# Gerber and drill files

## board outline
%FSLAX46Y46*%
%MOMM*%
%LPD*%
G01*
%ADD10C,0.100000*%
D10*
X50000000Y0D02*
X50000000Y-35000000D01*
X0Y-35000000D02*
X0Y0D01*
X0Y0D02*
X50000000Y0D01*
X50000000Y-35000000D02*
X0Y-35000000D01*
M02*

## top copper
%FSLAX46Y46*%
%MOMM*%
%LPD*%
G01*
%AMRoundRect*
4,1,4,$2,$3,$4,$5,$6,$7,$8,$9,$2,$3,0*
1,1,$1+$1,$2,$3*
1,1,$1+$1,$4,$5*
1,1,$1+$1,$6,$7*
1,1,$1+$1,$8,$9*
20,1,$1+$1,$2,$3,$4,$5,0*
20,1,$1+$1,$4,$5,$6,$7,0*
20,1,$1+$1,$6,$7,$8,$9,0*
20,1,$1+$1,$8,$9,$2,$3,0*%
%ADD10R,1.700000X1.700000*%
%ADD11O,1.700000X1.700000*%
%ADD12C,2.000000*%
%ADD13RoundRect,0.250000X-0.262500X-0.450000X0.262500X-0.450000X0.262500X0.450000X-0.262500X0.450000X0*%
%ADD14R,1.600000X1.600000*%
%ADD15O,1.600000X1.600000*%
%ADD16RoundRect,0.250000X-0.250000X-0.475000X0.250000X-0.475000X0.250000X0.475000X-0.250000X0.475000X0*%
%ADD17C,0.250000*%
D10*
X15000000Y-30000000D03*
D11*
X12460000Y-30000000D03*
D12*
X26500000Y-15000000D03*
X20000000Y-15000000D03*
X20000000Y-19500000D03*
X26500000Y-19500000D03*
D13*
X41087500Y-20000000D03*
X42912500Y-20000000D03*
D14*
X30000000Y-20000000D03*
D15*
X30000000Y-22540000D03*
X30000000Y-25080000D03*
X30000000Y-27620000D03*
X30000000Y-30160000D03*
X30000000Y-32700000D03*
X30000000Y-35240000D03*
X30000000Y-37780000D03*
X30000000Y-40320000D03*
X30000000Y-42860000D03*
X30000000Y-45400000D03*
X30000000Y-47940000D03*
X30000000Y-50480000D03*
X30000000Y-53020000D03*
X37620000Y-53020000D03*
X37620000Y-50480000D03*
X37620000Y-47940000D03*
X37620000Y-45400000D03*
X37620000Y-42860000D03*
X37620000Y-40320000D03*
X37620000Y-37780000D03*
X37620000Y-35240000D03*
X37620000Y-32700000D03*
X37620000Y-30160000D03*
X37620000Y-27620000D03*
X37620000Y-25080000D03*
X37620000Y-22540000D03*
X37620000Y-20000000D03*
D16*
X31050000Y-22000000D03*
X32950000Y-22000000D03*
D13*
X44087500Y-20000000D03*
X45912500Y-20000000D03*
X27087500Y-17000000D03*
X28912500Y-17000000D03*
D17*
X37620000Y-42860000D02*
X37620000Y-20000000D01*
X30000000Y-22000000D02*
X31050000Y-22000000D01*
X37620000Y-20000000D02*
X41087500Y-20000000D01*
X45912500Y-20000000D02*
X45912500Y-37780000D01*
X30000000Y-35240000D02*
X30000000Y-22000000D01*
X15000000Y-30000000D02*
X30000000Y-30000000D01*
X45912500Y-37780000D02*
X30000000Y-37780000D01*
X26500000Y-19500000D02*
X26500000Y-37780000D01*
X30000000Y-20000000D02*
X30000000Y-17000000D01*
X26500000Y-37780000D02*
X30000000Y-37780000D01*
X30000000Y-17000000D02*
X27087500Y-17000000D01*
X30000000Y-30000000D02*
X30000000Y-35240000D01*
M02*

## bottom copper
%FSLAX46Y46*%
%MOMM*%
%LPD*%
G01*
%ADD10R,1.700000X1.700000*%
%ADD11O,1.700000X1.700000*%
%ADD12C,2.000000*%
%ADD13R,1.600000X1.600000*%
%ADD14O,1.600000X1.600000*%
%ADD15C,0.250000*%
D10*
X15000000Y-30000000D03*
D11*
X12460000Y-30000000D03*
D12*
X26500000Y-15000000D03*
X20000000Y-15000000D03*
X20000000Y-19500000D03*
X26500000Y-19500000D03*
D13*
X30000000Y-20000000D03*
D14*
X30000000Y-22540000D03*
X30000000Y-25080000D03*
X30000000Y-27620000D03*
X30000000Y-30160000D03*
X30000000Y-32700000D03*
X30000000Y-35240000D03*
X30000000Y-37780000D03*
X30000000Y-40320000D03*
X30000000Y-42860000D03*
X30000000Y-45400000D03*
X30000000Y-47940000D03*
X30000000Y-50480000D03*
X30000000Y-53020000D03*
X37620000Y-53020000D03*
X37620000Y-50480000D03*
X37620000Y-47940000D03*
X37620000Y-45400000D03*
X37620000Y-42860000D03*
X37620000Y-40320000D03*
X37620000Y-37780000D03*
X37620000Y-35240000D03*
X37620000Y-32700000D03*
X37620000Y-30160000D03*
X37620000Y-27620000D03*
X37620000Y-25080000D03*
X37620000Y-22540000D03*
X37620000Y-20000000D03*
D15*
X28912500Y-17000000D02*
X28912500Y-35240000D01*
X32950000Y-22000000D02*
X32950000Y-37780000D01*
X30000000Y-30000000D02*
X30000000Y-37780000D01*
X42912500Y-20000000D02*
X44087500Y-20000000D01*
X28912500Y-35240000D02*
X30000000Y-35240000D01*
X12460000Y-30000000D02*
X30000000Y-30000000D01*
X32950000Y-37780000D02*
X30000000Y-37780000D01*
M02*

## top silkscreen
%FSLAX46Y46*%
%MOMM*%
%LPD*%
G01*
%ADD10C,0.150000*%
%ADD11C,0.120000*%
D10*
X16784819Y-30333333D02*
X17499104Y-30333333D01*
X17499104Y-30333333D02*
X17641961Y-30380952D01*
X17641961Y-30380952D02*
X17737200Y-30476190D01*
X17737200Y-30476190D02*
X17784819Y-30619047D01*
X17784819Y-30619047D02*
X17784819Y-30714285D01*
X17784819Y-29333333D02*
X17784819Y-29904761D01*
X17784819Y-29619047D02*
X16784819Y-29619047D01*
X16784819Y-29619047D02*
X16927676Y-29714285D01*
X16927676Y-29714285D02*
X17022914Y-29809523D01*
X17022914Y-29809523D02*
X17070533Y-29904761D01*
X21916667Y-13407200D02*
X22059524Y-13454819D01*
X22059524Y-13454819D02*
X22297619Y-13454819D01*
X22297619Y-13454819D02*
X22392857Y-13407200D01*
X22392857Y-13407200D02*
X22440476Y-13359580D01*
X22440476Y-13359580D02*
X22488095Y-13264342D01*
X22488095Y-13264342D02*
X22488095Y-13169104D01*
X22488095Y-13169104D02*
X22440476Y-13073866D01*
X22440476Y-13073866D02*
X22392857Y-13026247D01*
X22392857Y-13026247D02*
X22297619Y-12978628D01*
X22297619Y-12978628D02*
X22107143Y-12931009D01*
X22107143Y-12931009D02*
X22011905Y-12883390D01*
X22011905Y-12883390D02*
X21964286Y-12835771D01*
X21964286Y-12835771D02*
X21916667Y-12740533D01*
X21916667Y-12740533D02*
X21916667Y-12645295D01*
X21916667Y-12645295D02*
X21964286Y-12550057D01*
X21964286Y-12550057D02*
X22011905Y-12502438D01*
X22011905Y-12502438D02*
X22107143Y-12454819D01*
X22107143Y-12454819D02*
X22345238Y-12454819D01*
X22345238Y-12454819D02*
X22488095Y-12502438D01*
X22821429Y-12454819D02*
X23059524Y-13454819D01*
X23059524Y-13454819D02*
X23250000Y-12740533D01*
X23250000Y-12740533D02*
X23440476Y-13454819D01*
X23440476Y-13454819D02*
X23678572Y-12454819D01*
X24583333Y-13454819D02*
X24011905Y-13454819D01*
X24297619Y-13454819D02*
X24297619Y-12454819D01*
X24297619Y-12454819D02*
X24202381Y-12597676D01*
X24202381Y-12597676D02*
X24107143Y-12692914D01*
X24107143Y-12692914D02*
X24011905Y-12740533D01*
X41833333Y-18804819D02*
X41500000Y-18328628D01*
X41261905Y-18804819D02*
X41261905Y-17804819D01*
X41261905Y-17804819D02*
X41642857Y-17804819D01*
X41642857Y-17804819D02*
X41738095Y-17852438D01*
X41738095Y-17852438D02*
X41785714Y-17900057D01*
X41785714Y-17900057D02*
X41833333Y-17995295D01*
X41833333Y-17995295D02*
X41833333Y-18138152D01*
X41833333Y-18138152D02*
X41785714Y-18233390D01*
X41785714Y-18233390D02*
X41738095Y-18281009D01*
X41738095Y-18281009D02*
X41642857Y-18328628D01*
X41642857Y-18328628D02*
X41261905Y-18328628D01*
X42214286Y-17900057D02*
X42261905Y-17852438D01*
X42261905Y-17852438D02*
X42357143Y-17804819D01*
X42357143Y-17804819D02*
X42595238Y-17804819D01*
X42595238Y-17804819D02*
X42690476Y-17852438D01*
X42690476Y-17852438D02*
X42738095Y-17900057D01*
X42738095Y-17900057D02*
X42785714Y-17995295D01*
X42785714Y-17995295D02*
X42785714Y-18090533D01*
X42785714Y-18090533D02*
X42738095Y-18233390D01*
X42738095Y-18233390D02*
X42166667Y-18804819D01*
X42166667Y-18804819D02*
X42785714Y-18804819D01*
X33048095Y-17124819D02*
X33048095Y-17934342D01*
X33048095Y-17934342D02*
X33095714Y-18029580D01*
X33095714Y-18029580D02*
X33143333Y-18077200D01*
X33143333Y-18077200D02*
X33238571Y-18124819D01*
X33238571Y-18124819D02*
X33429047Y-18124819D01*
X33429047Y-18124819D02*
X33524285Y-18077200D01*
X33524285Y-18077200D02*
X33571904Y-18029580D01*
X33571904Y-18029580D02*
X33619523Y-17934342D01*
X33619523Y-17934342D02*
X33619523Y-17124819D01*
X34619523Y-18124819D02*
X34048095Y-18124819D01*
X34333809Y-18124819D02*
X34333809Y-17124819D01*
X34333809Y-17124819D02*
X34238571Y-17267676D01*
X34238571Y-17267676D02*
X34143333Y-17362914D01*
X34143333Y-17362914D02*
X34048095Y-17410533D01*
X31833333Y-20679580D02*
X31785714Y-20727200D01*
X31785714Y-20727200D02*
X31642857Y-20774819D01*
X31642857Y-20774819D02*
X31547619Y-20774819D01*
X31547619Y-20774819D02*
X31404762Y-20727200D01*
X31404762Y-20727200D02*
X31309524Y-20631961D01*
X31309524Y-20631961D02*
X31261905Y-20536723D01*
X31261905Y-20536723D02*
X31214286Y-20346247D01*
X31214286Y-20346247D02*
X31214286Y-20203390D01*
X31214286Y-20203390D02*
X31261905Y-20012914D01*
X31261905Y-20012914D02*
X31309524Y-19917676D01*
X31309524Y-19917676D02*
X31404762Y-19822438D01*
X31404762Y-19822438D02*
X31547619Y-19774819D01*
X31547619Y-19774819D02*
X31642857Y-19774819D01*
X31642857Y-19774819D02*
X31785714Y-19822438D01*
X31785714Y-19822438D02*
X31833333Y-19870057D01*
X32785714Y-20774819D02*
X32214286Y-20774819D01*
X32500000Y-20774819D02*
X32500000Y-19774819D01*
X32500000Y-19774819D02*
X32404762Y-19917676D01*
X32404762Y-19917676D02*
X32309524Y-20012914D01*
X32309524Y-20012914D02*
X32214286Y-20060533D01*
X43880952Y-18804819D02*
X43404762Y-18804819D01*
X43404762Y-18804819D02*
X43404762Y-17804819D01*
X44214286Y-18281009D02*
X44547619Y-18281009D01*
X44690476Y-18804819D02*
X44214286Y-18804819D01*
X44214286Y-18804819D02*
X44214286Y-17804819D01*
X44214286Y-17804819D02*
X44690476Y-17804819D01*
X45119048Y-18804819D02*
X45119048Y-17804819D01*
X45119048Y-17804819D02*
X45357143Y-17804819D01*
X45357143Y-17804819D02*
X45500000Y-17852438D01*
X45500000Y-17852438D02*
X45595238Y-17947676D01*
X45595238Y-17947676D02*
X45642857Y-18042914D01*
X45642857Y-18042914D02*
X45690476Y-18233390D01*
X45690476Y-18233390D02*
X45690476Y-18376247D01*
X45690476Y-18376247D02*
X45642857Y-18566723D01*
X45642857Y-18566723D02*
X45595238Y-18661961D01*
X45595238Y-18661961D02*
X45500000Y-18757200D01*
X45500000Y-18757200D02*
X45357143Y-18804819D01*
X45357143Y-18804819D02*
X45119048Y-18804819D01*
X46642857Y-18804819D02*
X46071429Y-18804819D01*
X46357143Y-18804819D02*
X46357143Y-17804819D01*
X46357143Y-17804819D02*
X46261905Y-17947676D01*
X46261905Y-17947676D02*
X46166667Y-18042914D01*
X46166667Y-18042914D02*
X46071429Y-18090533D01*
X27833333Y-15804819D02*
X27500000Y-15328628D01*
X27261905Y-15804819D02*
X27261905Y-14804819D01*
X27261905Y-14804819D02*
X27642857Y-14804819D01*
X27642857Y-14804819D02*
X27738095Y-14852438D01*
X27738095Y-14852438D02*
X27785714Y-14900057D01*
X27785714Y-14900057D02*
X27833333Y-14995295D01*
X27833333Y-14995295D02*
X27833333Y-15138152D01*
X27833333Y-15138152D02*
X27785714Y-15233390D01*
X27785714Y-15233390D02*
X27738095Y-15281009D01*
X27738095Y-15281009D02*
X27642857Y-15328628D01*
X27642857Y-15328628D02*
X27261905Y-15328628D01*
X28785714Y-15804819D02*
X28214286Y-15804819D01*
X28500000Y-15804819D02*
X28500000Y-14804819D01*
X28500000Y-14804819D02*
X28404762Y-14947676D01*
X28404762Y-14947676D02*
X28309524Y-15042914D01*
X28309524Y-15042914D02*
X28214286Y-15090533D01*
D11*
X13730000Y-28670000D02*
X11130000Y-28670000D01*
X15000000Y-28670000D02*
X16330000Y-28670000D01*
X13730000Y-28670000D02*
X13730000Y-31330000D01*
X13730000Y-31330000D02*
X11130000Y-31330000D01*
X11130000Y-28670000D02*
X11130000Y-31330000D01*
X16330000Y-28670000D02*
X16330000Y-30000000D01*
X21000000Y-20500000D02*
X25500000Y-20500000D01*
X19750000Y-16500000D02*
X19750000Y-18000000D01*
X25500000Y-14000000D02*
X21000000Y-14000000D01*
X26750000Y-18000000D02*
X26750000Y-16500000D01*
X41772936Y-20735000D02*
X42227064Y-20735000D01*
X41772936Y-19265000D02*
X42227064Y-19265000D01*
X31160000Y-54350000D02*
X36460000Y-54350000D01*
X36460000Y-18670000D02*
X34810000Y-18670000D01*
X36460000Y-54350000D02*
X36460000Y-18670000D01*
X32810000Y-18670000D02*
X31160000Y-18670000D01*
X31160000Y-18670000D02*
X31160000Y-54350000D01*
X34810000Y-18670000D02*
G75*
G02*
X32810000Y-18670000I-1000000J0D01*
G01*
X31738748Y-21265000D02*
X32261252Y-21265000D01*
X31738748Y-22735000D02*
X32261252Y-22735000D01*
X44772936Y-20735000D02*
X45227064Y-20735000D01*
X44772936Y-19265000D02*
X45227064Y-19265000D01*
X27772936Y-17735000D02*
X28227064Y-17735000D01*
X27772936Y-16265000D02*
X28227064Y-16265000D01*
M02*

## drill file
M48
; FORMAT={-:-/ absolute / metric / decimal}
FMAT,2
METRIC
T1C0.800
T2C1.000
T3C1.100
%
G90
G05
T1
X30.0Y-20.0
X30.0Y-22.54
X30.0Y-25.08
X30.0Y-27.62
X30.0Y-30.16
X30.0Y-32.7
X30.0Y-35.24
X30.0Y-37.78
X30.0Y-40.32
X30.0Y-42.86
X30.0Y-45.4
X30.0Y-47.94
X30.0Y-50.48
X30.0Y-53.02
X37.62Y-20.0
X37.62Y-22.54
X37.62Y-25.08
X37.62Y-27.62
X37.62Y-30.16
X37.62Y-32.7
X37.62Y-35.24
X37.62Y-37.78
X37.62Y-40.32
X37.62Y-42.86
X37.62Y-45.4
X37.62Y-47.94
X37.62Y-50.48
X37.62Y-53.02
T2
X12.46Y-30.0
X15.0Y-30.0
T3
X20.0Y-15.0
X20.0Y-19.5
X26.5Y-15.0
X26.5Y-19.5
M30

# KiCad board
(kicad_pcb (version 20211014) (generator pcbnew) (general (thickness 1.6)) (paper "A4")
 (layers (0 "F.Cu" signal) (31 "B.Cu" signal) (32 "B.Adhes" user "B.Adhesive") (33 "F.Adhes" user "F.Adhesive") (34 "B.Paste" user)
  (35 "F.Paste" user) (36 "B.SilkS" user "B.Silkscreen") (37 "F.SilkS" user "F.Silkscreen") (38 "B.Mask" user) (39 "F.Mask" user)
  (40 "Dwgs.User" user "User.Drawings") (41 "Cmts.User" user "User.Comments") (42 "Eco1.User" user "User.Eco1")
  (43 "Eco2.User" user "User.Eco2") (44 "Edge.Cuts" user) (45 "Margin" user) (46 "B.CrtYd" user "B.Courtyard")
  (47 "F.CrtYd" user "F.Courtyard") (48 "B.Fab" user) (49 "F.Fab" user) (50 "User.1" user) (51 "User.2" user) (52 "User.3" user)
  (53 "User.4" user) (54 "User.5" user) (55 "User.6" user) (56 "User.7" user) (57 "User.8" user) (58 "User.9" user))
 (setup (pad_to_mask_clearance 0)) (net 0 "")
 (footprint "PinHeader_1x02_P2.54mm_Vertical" (layer "F.Cu") (at 15 30 -90)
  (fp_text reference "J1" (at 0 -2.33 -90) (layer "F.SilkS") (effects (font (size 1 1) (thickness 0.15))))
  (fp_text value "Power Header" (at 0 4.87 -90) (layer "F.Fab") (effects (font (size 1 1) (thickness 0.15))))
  (fp_line (start -1.33 1.27) (end -1.33 3.87) (layer "F.SilkS") (width 0.12))
  (fp_line (start -1.33 0) (end -1.33 -1.33) (layer "F.SilkS") (width 0.12))
  (fp_line (start -1.33 1.27) (end 1.33 1.27) (layer "F.SilkS") (width 0.12))
  (fp_line (start 1.33 1.27) (end 1.33 3.87) (layer "F.SilkS") (width 0.12))
  (fp_line (start -1.33 3.87) (end 1.33 3.87) (layer "F.SilkS") (width 0.12))
  (fp_line (start -1.33 -1.33) (end 0 -1.33) (layer "F.SilkS") (width 0.12))
  (pad "1" thru_hole rect (at 0 0 270) (size 1.7 1.7) (drill 1) (layers *.Cu *.Mask))
  (pad "2" thru_hole oval (at 0 2.54 270) (size 1.7 1.7) (drill 1) (layers *.Cu *.Mask)))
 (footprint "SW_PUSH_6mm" (layer "F.Cu") (at 20 15)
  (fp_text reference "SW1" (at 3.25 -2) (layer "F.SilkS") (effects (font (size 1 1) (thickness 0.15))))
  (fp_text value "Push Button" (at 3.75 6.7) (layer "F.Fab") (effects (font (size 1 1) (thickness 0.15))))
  (fp_line (start 1 5.5) (end 5.5 5.5) (layer "F.SilkS") (width 0.12))
  (fp_line (start -0.25 1.5) (end -0.25 3) (layer "F.SilkS") (width 0.12))
  (fp_line (start 5.5 -1) (end 1 -1) (layer "F.SilkS") (width 0.12))
  (fp_line (start 6.75 3) (end 6.75 1.5) (layer "F.SilkS") (width 0.12))
  (pad "1" thru_hole circle (at 6.5 0 90) (size 2 2) (drill 1.1) (layers *.Cu *.Mask))
  (pad "1" thru_hole circle (at 0 0 90) (size 2 2) (drill 1.1) (layers *.Cu *.Mask))
  (pad "2" thru_hole circle (at 0 4.5 90) (size 2 2) (drill 1.1) (layers *.Cu *.Mask))
  (pad "2" thru_hole circle (at 6.5 4.5 90) (size 2 2) (drill 1.1) (layers *.Cu *.Mask)))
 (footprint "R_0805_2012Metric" (layer "F.Cu") (at 42 20)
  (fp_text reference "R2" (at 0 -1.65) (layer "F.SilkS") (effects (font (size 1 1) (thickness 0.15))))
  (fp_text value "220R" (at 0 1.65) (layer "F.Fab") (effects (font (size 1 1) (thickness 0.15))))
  (fp_line (start -0.227064 0.735) (end 0.227064 0.735) (layer "F.SilkS") (width 0.12))
  (fp_line (start -0.227064 -0.735) (end 0.227064 -0.735) (layer "F.SilkS") (width 0.12))
  (pad "1" smd roundrect (at -0.9125 0) (size 1.025 1.4) (layers "F.Cu" "F.Paste" "F.Mask") (roundrect_rratio 0.243902))
  (pad "2" smd roundrect (at 0.9125 0) (size 1.025 1.4) (layers "F.Cu" "F.Paste" "F.Mask") (roundrect_rratio 0.243902)))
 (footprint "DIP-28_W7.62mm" (layer "F.Cu") (at 30 20)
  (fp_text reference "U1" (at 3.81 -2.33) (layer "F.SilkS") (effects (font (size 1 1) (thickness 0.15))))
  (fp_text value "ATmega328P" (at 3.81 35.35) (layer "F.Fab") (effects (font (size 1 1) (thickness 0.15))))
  (fp_line (start 1.16 34.35) (end 6.46 34.35) (layer "F.SilkS") (width 0.12))
  (fp_line (start 6.46 -1.33) (end 4.81 -1.33) (layer "F.SilkS") (width 0.12))
  (fp_line (start 6.46 34.35) (end 6.46 -1.33) (layer "F.SilkS") (width 0.12))
  (fp_line (start 2.81 -1.33) (end 1.16 -1.33) (layer "F.SilkS") (width 0.12))
  (fp_line (start 1.16 -1.33) (end 1.16 34.35) (layer "F.SilkS") (width 0.12))
  (fp_arc (start 4.81 -1.33) (mid 3.81 -0.33) (end 2.81 -1.33) (layer "F.SilkS") (width 0.12))
  (pad "1" thru_hole rect (at 0 0) (size 1.6 1.6) (drill 0.8) (layers *.Cu *.Mask))
  (pad "2" thru_hole oval (at 0 2.54) (size 1.6 1.6) (drill 0.8) (layers *.Cu *.Mask))
  (pad "3" thru_hole oval (at 0 5.08) (size 1.6 1.6) (drill 0.8) (layers *.Cu *.Mask))
  (pad "4" thru_hole oval (at 0 7.62) (size 1.6 1.6) (drill 0.8) (layers *.Cu *.Mask))
  (pad "5" thru_hole oval (at 0 10.16) (size 1.6 1.6) (drill 0.8) (layers *.Cu *.Mask))
  (pad "6" thru_hole oval (at 0 12.7) (size 1.6 1.6) (drill 0.8) (layers *.Cu *.Mask))
  (pad "7" thru_hole oval (at 0 15.24) (size 1.6 1.6) (drill 0.8) (layers *.Cu *.Mask))
  (pad "8" thru_hole oval (at 0 17.78) (size 1.6 1.6) (drill 0.8) (layers *.Cu *.Mask))
  (pad "9" thru_hole oval (at 0 20.32) (size 1.6 1.6) (drill 0.8) (layers *.Cu *.Mask))
  (pad "10" thru_hole oval (at 0 22.86) (size 1.6 1.6) (drill 0.8) (layers *.Cu *.Mask))
  (pad "11" thru_hole oval (at 0 25.4) (size 1.6 1.6) (drill 0.8) (layers *.Cu *.Mask))
  (pad "12" thru_hole oval (at 0 27.94) (size 1.6 1.6) (drill 0.8) (layers *.Cu *.Mask))
  (pad "13" thru_hole oval (at 0 30.48) (size 1.6 1.6) (drill 0.8) (layers *.Cu *.Mask))
  (pad "14" thru_hole oval (at 0 33.02) (size 1.6 1.6) (drill 0.8) (layers *.Cu *.Mask))
  (pad "15" thru_hole oval (at 7.62 33.02) (size 1.6 1.6) (drill 0.8) (layers *.Cu *.Mask))
  (pad "16" thru_hole oval (at 7.62 30.48) (size 1.6 1.6) (drill 0.8) (layers *.Cu *.Mask))
  (pad "17" thru_hole oval (at 7.62 27.94) (size 1.6 1.6) (drill 0.8) (layers *.Cu *.Mask))
  (pad "18" thru_hole oval (at 7.62 25.4) (size 1.6 1.6) (drill 0.8) (layers *.Cu *.Mask))
  (pad "19" thru_hole oval (at 7.62 22.86) (size 1.6 1.6) (drill 0.8) (layers *.Cu *.Mask))
  (pad "20" thru_hole oval (at 7.62 20.32) (size 1.6 1.6) (drill 0.8) (layers *.Cu *.Mask))
  (pad "21" thru_hole oval (at 7.62 17.78) (size 1.6 1.6) (drill 0.8) (layers *.Cu *.Mask))
  (pad "22" thru_hole oval (at 7.62 15.24) (size 1.6 1.6) (drill 0.8) (layers *.Cu *.Mask))
  (pad "23" thru_hole oval (at 7.62 12.7) (size 1.6 1.6) (drill 0.8) (layers *.Cu *.Mask))
  (pad "24" thru_hole oval (at 7.62 10.16) (size 1.6 1.6) (drill 0.8) (layers *.Cu *.Mask))
  (pad "25" thru_hole oval (at 7.62 7.62) (size 1.6 1.6) (drill 0.8) (layers *.Cu *.Mask))
  (pad "26" thru_hole oval (at 7.62 5.08) (size 1.6 1.6) (drill 0.8) (layers *.Cu *.Mask))
  (pad "27" thru_hole oval (at 7.62 2.54) (size 1.6 1.6) (drill 0.8) (layers *.Cu *.Mask))
  (pad "28" thru_hole oval (at 7.62 0) (size 1.6 1.6) (drill 0.8) (layers *.Cu *.Mask)))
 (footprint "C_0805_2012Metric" (layer "F.Cu") (at 32 22)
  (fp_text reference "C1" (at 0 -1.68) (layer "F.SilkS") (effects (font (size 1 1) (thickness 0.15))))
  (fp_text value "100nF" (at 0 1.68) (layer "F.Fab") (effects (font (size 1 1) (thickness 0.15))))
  (fp_line (start -0.261252 -0.735) (end 0.261252 -0.735) (layer "F.SilkS") (width 0.12))
  (fp_line (start -0.261252 0.735) (end 0.261252 0.735) (layer "F.SilkS") (width 0.12))
  (pad "1" smd roundrect (at -0.95 0) (size 1 1.45) (layers "F.Cu" "F.Paste" "F.Mask") (roundrect_rratio 0.25))
  (pad "2" smd roundrect (at 0.95 0) (size 1 1.45) (layers "F.Cu" "F.Paste" "F.Mask") (roundrect_rratio 0.25)))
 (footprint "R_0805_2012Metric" (layer "F.Cu") (at 45 20)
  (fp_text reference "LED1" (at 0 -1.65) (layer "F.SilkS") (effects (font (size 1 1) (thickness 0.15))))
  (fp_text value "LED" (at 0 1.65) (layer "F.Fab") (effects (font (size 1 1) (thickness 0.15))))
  (fp_line (start -0.227064 0.735) (end 0.227064 0.735) (layer "F.SilkS") (width 0.12))
  (fp_line (start -0.227064 -0.735) (end 0.227064 -0.735) (layer "F.SilkS") (width 0.12))
  (pad "1" smd roundrect (at -0.9125 0) (size 1.025 1.4) (layers "F.Cu" "F.Paste" "F.Mask") (roundrect_rratio 0.243902))
  (pad "2" smd roundrect (at 0.9125 0) (size 1.025 1.4) (layers "F.Cu" "F.Paste" "F.Mask") (roundrect_rratio 0.243902)))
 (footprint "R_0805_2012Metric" (layer "F.Cu") (at 28 17)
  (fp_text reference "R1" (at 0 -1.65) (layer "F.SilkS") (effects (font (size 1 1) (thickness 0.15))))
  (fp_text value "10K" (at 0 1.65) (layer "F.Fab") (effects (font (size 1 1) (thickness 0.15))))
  (fp_line (start -0.227064 0.735) (end 0.227064 0.735) (layer "F.SilkS") (width 0.12))
  (fp_line (start -0.227064 -0.735) (end 0.227064 -0.735) (layer "F.SilkS") (width 0.12))
  (pad "1" smd roundrect (at -0.9125 0) (size 1.025 1.4) (layers "F.Cu" "F.Paste" "F.Mask") (roundrect_rratio 0.243902))
  (pad "2" smd roundrect (at 0.9125 0) (size 1.025 1.4) (layers "F.Cu" "F.Paste" "F.Mask") (roundrect_rratio 0.243902)))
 (gr_line (start 50 0) (end 50 35) (layer "Edge.Cuts") (width 0.1))
 (gr_line (start 0 35) (end 0 0) (layer "Edge.Cuts") (width 0.1))
 (gr_line (start 0 0) (end 50 0) (layer "Edge.Cuts") (width 0.1))
 (gr_line (start 50 35) (end 0 35) (layer "Edge.Cuts") (width 0.1))
 (segment (start 37.62 42.86) (end 37.62 20) (width 0.25) (layer "F.Cu") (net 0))
 (segment (start 30 22) (end 31.05 22) (width 0.25) (layer "F.Cu") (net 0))
 (segment (start 37.62 20) (end 41.0875 20) (width 0.25) (layer "F.Cu") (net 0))
 (segment (start 45.9125 20) (end 45.9125 37.78) (width 0.25) (layer "F.Cu") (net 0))
 (segment (start 30 35.24) (end 30 22) (width 0.25) (layer "F.Cu") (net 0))
 (segment (start 15 30) (end 30 30) (width 0.25) (layer "F.Cu") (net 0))
 (segment (start 45.9125 37.78) (end 30 37.78) (width 0.25) (layer "F.Cu") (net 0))
 (segment (start 26.5 19.5) (end 26.5 37.78) (width 0.25) (layer "F.Cu") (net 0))
 (segment (start 30 20) (end 30 17) (width 0.25) (layer "F.Cu") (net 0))
 (segment (start 26.5 37.78) (end 30 37.78) (width 0.25) (layer "F.Cu") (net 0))
 (segment (start 30 17) (end 27.0875 17) (width 0.25) (layer "F.Cu") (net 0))
 (segment (start 30 30) (end 30 35.24) (width 0.25) (layer "F.Cu") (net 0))
 (segment (start 28.9125 17) (end 28.9125 35.24) (width 0.25) (layer "B.Cu") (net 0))
 (segment (start 32.95 22) (end 32.95 37.78) (width 0.25) (layer "B.Cu") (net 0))
 (segment (start 30 30) (end 30 37.78) (width 0.25) (layer "B.Cu") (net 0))
 (segment (start 42.9125 20) (end 44.0875 20) (width 0.25) (layer "B.Cu") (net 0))
 (segment (start 28.9125 35.24) (end 30 35.24) (width 0.25) (layer "B.Cu") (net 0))
 (segment (start 12.46 30) (end 30 30) (width 0.25) (layer "B.Cu") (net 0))
 (segment (start 32.95 37.78) (end 30 37.78) (width 0.25) (layer "B.Cu") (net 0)))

